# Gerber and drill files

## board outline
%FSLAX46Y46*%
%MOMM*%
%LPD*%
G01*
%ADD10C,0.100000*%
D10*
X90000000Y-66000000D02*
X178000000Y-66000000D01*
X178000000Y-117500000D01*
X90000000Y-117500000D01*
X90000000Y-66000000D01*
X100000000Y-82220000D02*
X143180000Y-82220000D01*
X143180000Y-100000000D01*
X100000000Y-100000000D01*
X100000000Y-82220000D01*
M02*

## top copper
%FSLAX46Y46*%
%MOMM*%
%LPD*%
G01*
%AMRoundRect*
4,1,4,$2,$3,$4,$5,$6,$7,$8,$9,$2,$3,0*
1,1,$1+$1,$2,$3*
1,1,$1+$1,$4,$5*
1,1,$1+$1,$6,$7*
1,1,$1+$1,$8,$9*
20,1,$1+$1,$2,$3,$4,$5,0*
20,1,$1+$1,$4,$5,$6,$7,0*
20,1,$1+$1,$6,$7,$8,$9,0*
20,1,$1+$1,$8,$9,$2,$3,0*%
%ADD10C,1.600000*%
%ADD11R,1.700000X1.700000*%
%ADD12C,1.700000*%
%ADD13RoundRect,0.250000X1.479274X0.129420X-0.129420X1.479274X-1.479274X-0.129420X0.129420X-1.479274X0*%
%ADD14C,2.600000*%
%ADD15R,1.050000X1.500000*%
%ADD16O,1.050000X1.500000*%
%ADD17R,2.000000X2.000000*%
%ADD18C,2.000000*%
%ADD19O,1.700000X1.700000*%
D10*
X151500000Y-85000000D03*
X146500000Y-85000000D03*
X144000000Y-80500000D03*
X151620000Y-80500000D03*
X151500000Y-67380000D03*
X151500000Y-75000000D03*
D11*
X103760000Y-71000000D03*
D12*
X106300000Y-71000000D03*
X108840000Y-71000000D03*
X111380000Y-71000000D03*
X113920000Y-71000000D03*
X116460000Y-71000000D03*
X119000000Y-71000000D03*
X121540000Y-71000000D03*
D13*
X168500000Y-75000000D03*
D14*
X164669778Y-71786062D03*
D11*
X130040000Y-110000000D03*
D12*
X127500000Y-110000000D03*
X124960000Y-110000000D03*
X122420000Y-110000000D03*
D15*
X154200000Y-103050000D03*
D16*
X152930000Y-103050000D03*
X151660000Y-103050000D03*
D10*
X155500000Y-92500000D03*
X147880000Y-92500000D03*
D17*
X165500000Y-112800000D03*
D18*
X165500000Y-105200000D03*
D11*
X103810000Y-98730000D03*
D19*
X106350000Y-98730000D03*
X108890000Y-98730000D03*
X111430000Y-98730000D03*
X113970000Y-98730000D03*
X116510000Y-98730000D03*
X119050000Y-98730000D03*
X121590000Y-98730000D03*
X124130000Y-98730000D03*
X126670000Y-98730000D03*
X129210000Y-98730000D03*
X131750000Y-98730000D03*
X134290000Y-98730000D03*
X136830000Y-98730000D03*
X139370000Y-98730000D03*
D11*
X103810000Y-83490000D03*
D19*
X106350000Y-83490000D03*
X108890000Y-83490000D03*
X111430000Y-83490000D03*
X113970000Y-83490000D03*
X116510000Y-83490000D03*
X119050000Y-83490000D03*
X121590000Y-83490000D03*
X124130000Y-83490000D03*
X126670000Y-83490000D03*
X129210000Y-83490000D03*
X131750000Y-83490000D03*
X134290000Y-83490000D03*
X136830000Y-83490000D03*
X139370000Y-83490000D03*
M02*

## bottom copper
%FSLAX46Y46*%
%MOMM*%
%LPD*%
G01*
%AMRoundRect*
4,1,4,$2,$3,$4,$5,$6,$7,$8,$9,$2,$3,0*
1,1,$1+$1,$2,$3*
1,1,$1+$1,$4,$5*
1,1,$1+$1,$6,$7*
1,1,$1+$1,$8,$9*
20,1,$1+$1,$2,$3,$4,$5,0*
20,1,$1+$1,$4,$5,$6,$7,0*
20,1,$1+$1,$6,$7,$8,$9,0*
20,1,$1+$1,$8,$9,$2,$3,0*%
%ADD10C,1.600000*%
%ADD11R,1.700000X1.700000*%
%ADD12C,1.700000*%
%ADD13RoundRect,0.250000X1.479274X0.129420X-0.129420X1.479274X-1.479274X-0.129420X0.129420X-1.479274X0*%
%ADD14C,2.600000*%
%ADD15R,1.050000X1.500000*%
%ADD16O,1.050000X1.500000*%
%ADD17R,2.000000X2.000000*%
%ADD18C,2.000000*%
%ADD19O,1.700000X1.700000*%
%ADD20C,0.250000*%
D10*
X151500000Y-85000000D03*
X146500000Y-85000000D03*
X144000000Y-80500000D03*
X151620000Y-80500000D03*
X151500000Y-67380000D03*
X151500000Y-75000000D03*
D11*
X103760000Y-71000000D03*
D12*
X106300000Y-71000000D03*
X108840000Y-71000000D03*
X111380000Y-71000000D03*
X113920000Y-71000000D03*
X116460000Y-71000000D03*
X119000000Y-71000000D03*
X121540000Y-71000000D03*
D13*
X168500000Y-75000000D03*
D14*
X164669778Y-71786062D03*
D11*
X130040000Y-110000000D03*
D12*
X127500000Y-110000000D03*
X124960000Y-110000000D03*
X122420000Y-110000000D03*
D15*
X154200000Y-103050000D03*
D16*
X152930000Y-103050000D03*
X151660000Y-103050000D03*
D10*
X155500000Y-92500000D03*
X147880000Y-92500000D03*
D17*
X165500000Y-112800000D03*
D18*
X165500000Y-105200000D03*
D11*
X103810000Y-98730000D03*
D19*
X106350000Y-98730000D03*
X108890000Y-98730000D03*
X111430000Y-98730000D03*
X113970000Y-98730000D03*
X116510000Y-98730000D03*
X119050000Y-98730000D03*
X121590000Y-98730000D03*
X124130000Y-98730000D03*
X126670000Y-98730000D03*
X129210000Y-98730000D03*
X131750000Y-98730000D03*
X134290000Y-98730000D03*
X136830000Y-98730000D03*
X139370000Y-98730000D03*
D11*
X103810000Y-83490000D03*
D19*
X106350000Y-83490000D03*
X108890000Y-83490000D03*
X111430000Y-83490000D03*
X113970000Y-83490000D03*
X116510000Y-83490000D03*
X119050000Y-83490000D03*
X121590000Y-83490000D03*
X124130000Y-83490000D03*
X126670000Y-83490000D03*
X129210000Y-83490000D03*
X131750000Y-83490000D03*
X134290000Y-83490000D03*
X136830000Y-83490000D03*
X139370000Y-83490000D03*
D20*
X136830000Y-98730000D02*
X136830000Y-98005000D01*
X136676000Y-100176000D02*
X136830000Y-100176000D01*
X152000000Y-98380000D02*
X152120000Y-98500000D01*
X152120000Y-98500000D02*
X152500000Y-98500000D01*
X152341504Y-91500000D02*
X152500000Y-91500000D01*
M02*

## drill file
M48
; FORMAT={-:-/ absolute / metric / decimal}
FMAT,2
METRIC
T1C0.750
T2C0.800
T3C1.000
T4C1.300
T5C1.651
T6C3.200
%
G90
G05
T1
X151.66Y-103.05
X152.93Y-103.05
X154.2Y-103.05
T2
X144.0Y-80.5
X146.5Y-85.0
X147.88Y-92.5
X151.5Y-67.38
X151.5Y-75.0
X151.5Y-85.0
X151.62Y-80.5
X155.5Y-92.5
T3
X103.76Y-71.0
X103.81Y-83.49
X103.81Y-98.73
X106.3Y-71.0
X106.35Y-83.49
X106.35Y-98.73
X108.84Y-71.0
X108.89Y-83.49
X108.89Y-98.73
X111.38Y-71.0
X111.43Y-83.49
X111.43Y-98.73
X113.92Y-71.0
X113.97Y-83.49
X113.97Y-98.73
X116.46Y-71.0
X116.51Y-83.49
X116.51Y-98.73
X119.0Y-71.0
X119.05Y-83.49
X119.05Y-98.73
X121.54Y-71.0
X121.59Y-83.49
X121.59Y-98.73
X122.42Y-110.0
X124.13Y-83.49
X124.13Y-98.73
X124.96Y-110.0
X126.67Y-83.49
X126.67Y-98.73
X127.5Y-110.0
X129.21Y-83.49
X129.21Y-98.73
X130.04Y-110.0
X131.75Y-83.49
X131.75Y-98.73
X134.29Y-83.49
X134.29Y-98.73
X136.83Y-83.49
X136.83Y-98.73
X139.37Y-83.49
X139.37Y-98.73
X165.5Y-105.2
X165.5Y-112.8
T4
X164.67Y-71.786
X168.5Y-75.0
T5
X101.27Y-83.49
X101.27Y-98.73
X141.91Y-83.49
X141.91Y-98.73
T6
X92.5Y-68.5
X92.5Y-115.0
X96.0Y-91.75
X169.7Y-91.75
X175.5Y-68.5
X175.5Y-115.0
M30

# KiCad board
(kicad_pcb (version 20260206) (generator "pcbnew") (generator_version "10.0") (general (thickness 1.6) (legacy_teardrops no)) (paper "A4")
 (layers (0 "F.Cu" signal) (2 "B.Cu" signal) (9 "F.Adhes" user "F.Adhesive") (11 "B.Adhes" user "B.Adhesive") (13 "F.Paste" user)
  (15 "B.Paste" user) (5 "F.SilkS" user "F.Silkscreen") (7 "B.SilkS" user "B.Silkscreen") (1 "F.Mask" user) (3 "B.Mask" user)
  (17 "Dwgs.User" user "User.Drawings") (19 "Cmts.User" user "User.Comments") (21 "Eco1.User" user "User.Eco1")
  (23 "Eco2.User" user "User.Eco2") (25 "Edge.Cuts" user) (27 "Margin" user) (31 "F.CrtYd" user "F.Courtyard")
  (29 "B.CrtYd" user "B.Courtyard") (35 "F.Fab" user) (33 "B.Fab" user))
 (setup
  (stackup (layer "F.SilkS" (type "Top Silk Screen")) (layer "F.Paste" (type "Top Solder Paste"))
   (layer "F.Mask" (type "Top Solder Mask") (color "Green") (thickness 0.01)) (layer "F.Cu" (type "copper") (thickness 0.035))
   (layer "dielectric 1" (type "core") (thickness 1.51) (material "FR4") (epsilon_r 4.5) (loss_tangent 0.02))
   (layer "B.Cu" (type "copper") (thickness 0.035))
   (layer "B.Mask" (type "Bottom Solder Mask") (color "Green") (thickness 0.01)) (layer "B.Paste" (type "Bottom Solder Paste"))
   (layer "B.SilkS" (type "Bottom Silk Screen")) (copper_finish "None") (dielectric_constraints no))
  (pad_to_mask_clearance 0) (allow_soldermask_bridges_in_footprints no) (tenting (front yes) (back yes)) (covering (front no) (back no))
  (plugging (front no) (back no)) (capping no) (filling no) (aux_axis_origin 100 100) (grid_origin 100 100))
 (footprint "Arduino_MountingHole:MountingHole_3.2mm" (layer "F.Cu") (at 96 91.75)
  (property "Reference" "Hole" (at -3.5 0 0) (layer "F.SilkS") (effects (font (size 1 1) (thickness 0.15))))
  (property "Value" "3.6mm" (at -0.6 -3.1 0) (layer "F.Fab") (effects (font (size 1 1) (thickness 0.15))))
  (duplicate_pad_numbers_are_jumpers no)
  (pad "" np_thru_hole circle (at 0 0) (size 3.2 3.2) (drill 3.2) (layers "*.Cu" "*.Mask")))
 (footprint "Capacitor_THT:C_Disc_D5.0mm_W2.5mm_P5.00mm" (layer "F.Cu") (at 151.5 85 180)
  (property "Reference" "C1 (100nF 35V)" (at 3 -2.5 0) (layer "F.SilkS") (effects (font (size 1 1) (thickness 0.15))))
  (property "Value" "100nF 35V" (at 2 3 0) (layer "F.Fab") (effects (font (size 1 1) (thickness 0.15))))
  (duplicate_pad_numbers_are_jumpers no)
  (pad "1" thru_hole circle (at 0 0 180) (size 1.6 1.6) (drill 0.8) (layers "*.Cu" "*.Mask") (remove_unused_layers no) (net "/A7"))
  (pad "2" thru_hole circle (at 5 0 180) (size 1.6 1.6) (drill 0.8) (layers "*.Cu" "*.Mask") (remove_unused_layers no) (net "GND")))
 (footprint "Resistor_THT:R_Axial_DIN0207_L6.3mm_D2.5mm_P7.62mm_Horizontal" (layer "F.Cu") (at 144 80.5)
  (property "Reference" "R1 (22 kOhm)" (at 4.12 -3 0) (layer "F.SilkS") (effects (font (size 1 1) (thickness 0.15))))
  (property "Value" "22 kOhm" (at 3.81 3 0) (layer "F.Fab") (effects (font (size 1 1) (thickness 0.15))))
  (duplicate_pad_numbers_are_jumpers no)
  (pad "1" thru_hole circle (at 0 0) (size 1.6 1.6) (drill 0.8) (layers "*.Cu" "*.Mask") (remove_unused_layers no) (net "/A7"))
  (pad "2" thru_hole circle (at 7.62 0) (size 1.6 1.6) (drill 0.8) (layers "*.Cu" "*.Mask") (remove_unused_layers no) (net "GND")))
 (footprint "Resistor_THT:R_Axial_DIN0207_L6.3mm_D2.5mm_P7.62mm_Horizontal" (layer "F.Cu") (at 151.5 67.38 -90)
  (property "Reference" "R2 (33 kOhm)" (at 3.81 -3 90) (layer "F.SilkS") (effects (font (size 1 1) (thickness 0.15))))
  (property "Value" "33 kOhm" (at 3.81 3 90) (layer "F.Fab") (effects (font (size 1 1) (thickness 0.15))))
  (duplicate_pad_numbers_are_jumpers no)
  (pad "1" thru_hole circle (at 0 0 270) (size 1.6 1.6) (drill 0.8) (layers "*.Cu" "*.Mask") (remove_unused_layers no) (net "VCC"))
  (pad "2" thru_hole circle (at 7.62 0 270) (size 1.6 1.6) (drill 0.8) (layers "*.Cu" "*.Mask") (remove_unused_layers no) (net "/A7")))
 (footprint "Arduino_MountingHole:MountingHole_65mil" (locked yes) (layer "F.Cu") (at 101.27 83.49)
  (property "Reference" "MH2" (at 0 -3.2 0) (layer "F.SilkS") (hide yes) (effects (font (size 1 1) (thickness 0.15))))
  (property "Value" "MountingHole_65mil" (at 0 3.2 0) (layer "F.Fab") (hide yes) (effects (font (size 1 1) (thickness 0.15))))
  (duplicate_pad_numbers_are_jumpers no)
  (pad "" np_thru_hole circle (at 0 0) (size 1.651 1.651) (drill 1.651) (layers "*.Cu" "*.Mask")))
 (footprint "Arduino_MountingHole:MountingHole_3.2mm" (layer "F.Cu") (at 92.5 115)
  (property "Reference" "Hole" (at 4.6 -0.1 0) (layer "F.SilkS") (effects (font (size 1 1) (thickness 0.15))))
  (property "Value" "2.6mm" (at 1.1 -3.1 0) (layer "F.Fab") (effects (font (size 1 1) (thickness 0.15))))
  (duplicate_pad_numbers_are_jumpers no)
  (pad "" np_thru_hole circle (at 0 0) (size 3.2 3.2) (drill 3.2) (layers "*.Cu" "*.Mask")))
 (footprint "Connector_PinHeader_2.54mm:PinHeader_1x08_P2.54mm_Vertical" (layer "F.Cu") (at 103.76 71 90)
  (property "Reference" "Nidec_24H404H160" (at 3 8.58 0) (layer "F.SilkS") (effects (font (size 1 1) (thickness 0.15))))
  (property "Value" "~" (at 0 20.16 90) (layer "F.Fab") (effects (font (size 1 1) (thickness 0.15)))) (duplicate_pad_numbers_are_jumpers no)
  (pad "1" thru_hole rect (at 0 0 90) (size 1.7 1.7) (drill 1) (layers "*.Cu" "*.Mask") (remove_unused_layers no) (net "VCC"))
  (pad "2" thru_hole circle (at 0 2.54 90) (size 1.7 1.7) (drill 1) (layers "*.Cu" "*.Mask") (remove_unused_layers no) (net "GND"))
  (pad "3" thru_hole circle (at 0 5.08 90) (size 1.7 1.7) (drill 1) (layers "*.Cu" "*.Mask") (remove_unused_layers no) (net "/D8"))
  (pad "4" thru_hole circle (at 0 7.62 90) (size 1.7 1.7) (drill 1) (layers "*.Cu" "*.Mask") (remove_unused_layers no) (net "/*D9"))
  (pad "5" thru_hole circle (at 0 10.16 90) (size 1.7 1.7) (drill 1) (layers "*.Cu" "*.Mask") (remove_unused_layers no) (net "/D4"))
  (pad "6" thru_hole circle (at 0 12.7 90) (size 1.7 1.7) (drill 1) (layers "*.Cu" "*.Mask") (remove_unused_layers no)
   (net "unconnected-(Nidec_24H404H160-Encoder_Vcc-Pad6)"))
  (pad "7" thru_hole circle (at 0 15.24 90) (size 1.7 1.7) (drill 1) (layers "*.Cu" "*.Mask") (remove_unused_layers no)
   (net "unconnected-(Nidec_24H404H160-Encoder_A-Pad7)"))
  (pad "8" thru_hole circle (at 0 17.78 90) (size 1.7 1.7) (drill 1) (layers "*.Cu" "*.Mask") (remove_unused_layers no)
   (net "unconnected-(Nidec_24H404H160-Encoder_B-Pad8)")))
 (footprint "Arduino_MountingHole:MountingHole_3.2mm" (layer "F.Cu") (at 175.5 68.5)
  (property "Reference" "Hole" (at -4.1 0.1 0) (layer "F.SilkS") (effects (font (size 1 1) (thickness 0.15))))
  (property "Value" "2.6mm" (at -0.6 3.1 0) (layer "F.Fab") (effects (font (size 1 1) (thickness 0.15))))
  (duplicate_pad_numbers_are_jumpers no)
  (pad "" np_thru_hole circle (at 0 0) (size 3.2 3.2) (drill 3.2) (layers "*.Cu" "*.Mask")))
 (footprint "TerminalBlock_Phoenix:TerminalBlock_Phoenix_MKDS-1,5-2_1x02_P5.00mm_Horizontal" (layer "F.Cu") (at 168.5 75 140)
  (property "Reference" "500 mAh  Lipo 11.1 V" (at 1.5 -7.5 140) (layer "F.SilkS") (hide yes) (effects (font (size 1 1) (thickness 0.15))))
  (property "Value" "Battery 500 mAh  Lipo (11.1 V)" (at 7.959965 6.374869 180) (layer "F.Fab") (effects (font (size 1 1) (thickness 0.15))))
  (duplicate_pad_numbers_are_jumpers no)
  (pad "1" thru_hole roundrect (at 0 0 140) (size 2.6 2.6) (drill 1.3) (layers "*.Cu" "*.Mask") (remove_unused_layers no)
   (roundrect_rratio 0.096154) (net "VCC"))
  (pad "2" thru_hole circle (at 5 0 140) (size 2.6 2.6) (drill 1.3) (layers "*.Cu" "*.Mask") (remove_unused_layers no) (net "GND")))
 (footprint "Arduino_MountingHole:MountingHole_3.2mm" (layer "F.Cu") (at 175.5 115)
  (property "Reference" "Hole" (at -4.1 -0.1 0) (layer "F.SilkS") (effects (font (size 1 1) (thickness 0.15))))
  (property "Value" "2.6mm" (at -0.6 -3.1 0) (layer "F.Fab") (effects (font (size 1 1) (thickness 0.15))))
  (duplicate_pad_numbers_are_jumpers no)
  (pad "" np_thru_hole circle (at 0 0) (size 3.2 3.2) (drill 3.2) (layers "*.Cu" "*.Mask")))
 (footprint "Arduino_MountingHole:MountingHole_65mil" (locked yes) (layer "F.Cu") (at 141.91 98.73)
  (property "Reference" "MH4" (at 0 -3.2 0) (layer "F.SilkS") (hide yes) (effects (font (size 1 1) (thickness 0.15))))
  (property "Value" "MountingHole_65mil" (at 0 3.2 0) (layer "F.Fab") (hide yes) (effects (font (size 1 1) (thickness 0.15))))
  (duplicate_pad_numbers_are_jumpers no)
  (pad "" np_thru_hole circle (at 0 0) (size 1.651 1.651) (drill 1.651) (layers "*.Cu" "*.Mask")))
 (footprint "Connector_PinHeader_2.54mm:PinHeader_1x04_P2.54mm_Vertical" (layer "F.Cu") (at 130.04 110 -90)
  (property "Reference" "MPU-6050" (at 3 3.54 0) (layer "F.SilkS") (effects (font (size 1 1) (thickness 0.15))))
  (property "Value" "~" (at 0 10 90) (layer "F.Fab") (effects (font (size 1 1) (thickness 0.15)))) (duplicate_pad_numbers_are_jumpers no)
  (pad "1" thru_hole rect (at 0 0 270) (size 1.7 1.7) (drill 1) (layers "*.Cu" "*.Mask") (remove_unused_layers no) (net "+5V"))
  (pad "2" thru_hole circle (at 0 2.54 270) (size 1.7 1.7) (drill 1) (layers "*.Cu" "*.Mask") (remove_unused_layers no) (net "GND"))
  (pad "3" thru_hole circle (at 0 5.08 270) (size 1.7 1.7) (drill 1) (layers "*.Cu" "*.Mask") (remove_unused_layers no)
   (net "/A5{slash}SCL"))
  (pad "4" thru_hole circle (at 0 7.62 270) (size 1.7 1.7) (drill 1) (layers "*.Cu" "*.Mask") (remove_unused_layers no)
   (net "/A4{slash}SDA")))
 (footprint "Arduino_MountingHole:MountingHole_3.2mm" (layer "F.Cu") (at 169.7 91.75)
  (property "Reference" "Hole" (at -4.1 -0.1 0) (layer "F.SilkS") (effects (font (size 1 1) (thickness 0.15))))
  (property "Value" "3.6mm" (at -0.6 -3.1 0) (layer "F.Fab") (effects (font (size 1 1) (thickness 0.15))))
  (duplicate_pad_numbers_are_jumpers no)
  (pad "" np_thru_hole circle (at 0 0) (size 3.2 3.2) (drill 3.2) (layers "*.Cu" "*.Mask")))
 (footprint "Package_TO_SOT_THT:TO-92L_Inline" (layer "F.Cu") (at 154.2 103.05 180)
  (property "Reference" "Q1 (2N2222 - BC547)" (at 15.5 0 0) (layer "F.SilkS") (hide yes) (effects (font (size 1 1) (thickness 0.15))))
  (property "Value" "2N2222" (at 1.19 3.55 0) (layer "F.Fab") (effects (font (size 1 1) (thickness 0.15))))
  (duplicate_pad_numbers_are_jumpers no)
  (pad "1" thru_hole rect (at 0 0 180) (size 1.05 1.5) (drill 0.75) (layers "*.Cu" "*.Mask") (remove_unused_layers no) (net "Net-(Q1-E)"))
  (pad "2" thru_hole oval (at 1.27 0 180) (size 1.05 1.5) (drill 0.75) (layers "*.Cu" "*.Mask") (remove_unused_layers no) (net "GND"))
  (pad "3" thru_hole oval (at 2.54 0 180) (size 1.05 1.5) (drill 0.75) (layers "*.Cu" "*.Mask") (remove_unused_layers no)
   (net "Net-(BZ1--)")))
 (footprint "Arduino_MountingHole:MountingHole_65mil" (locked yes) (layer "F.Cu") (at 101.27 98.73)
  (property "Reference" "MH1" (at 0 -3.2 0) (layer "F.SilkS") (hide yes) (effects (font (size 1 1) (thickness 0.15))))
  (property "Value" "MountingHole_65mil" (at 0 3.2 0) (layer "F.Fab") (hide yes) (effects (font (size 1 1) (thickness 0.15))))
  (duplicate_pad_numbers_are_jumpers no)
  (pad "" np_thru_hole circle (at 0 0) (size 1.651 1.651) (drill 1.651) (layers "*.Cu" "*.Mask")))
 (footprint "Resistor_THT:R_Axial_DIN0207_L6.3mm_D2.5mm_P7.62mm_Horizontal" (layer "F.Cu") (at 155.5 92.5 180)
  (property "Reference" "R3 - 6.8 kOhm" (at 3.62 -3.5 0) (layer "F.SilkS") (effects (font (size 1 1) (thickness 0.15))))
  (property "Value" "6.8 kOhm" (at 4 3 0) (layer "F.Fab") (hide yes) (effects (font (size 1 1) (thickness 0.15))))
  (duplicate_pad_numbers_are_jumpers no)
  (pad "1" thru_hole circle (at 0 0 180) (size 1.6 1.6) (drill 0.8) (layers "*.Cu" "*.Mask") (remove_unused_layers no) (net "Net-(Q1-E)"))
  (pad "2" thru_hole circle (at 7.62 0 180) (size 1.6 1.6) (drill 0.8) (layers "*.Cu" "*.Mask") (remove_unused_layers no)
   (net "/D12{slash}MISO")))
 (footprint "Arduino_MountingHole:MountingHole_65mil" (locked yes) (layer "F.Cu") (at 141.91 83.49)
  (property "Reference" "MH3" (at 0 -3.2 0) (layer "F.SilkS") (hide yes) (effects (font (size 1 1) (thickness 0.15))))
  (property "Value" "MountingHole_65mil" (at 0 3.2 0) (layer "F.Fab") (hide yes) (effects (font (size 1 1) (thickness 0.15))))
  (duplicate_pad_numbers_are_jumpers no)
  (pad "" np_thru_hole circle (at 0 0) (size 1.651 1.651) (drill 1.651) (layers "*.Cu" "*.Mask")))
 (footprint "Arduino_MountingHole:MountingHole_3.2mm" (layer "F.Cu") (at 92.5 68.5)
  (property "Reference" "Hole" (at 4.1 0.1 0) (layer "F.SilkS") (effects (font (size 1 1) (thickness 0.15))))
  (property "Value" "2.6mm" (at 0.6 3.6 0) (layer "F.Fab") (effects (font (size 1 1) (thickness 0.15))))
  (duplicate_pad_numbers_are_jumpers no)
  (pad "" np_thru_hole circle (at 0 0) (size 3.2 3.2) (drill 3.2) (layers "*.Cu" "*.Mask")))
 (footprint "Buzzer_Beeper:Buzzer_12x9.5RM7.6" (layer "F.Cu") (at 165.5 112.8 90)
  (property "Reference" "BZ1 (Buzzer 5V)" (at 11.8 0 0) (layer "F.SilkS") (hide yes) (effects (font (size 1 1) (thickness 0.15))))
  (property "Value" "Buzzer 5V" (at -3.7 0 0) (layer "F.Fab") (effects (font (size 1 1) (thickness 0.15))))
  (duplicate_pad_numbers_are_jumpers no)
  (pad "1" thru_hole rect (at 0 0 90) (size 2 2) (drill 1) (layers "*.Cu" "*.Mask") (remove_unused_layers no) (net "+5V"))
  (pad "2" thru_hole circle (at 7.6 0 90) (size 2 2) (drill 1) (layers "*.Cu" "*.Mask") (remove_unused_layers no) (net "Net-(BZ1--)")))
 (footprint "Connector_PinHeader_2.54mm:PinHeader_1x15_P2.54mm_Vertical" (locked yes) (layer "B.Cu") (at 103.81 98.73 -90)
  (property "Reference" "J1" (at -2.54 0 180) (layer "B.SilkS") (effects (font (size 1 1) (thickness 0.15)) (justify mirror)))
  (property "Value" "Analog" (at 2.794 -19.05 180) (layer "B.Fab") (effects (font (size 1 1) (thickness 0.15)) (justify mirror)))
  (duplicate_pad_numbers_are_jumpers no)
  (pad "1" thru_hole rect (at 0 0 270) (size 1.7 1.7) (drill 1) (layers "*.Cu" "*.Mask") (remove_unused_layers no) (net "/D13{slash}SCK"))
  (pad "2" thru_hole oval (at 0 -2.54 270) (size 1.7 1.7) (drill 1) (layers "*.Cu" "*.Mask") (remove_unused_layers no) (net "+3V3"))
  (pad "3" thru_hole oval (at 0 -5.08 270) (size 1.7 1.7) (drill 1) (layers "*.Cu" "*.Mask") (remove_unused_layers no) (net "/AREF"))
  (pad "4" thru_hole oval (at 0 -7.62 270) (size 1.7 1.7) (drill 1) (layers "*.Cu" "*.Mask") (remove_unused_layers no) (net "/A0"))
  (pad "5" thru_hole oval (at 0 -10.16 270) (size 1.7 1.7) (drill 1) (layers "*.Cu" "*.Mask") (remove_unused_layers no) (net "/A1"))
  (pad "6" thru_hole oval (at 0 -12.7 270) (size 1.7 1.7) (drill 1) (layers "*.Cu" "*.Mask") (remove_unused_layers no) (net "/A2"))
  (pad "7" thru_hole oval (at 0 -15.24 270) (size 1.7 1.7) (drill 1) (layers "*.Cu" "*.Mask") (remove_unused_layers no) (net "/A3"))
  (pad "8" thru_hole oval (at 0 -17.78 270) (size 1.7 1.7) (drill 1) (layers "*.Cu" "*.Mask") (remove_unused_layers no)
   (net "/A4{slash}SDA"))
  (pad "9" thru_hole oval (at 0 -20.32 270) (size 1.7 1.7) (drill 1) (layers "*.Cu" "*.Mask") (remove_unused_layers no)
   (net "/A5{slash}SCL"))
  (pad "10" thru_hole oval (at 0 -22.86 270) (size 1.7 1.7) (drill 1) (layers "*.Cu" "*.Mask") (remove_unused_layers no) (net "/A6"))
  (pad "11" thru_hole oval (at 0 -25.4 270) (size 1.7 1.7) (drill 1) (layers "*.Cu" "*.Mask") (remove_unused_layers no) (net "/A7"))
  (pad "12" thru_hole oval (at 0 -27.94 270) (size 1.7 1.7) (drill 1) (layers "*.Cu" "*.Mask") (remove_unused_layers no) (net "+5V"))
  (pad "13" thru_hole oval (at 0 -30.48 270) (size 1.7 1.7) (drill 1) (layers "*.Cu" "*.Mask") (remove_unused_layers no) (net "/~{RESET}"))
  (pad "14" thru_hole oval (at 0 -33.02 270) (size 1.7 1.7) (drill 1) (layers "*.Cu" "*.Mask") (remove_unused_layers no) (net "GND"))
  (pad "15" thru_hole oval (at 0 -35.56 270) (size 1.7 1.7) (drill 1) (layers "*.Cu" "*.Mask") (remove_unused_layers no) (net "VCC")))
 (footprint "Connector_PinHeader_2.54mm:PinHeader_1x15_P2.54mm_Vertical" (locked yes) (layer "B.Cu") (at 103.81 83.49 -90)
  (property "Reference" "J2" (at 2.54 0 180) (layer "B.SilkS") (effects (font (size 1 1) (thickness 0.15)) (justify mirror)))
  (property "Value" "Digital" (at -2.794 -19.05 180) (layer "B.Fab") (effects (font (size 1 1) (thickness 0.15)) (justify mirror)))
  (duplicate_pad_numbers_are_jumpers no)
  (pad "1" thru_hole rect (at 0 0 270) (size 1.7 1.7) (drill 1) (layers "*.Cu" "*.Mask") (remove_unused_layers no) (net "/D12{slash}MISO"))
  (pad "2" thru_hole oval (at 0 -2.54 270) (size 1.7 1.7) (drill 1) (layers "*.Cu" "*.Mask") (remove_unused_layers no)
   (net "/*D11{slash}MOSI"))
  (pad "3" thru_hole oval (at 0 -5.08 270) (size 1.7 1.7) (drill 1) (layers "*.Cu" "*.Mask") (remove_unused_layers no)
   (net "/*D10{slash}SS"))
  (pad "4" thru_hole oval (at 0 -7.62 270) (size 1.7 1.7) (drill 1) (layers "*.Cu" "*.Mask") (remove_unused_layers no) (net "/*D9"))
  (pad "5" thru_hole oval (at 0 -10.16 270) (size 1.7 1.7) (drill 1) (layers "*.Cu" "*.Mask") (remove_unused_layers no) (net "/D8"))
  (pad "6" thru_hole oval (at 0 -12.7 270) (size 1.7 1.7) (drill 1) (layers "*.Cu" "*.Mask") (remove_unused_layers no) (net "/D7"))
  (pad "7" thru_hole oval (at 0 -15.24 270) (size 1.7 1.7) (drill 1) (layers "*.Cu" "*.Mask") (remove_unused_layers no) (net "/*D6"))
  (pad "8" thru_hole oval (at 0 -17.78 270) (size 1.7 1.7) (drill 1) (layers "*.Cu" "*.Mask") (remove_unused_layers no) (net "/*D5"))
  (pad "9" thru_hole oval (at 0 -20.32 270) (size 1.7 1.7) (drill 1) (layers "*.Cu" "*.Mask") (remove_unused_layers no) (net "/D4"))
  (pad "10" thru_hole oval (at 0 -22.86 270) (size 1.7 1.7) (drill 1) (layers "*.Cu" "*.Mask") (remove_unused_layers no) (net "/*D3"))
  (pad "11" thru_hole oval (at 0 -25.4 270) (size 1.7 1.7) (drill 1) (layers "*.Cu" "*.Mask") (remove_unused_layers no) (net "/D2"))
  (pad "12" thru_hole oval (at 0 -27.94 270) (size 1.7 1.7) (drill 1) (layers "*.Cu" "*.Mask") (remove_unused_layers no) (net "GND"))
  (pad "13" thru_hole oval (at 0 -30.48 270) (size 1.7 1.7) (drill 1) (layers "*.Cu" "*.Mask") (remove_unused_layers no) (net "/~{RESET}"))
  (pad "14" thru_hole oval (at 0 -33.02 270) (size 1.7 1.7) (drill 1) (layers "*.Cu" "*.Mask") (remove_unused_layers no)
   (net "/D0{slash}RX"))
  (pad "15" thru_hole oval (at 0 -35.56 270) (size 1.7 1.7) (drill 1) (layers "*.Cu" "*.Mask") (remove_unused_layers no)
   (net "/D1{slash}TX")))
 (gr_rect (start 90 66) (end 178 117.5) (stroke (width 0.1) (type solid)) (fill no) (layer "Edge.Cuts"))
 (gr_rect (start 100 82.22) (end 143.18 100) (stroke (width 0.1) (type solid)) (fill no) (layer "Edge.Cuts"))
 (segment (start 136.83 98.73) (end 136.83 98.005) (width 0.25) (layer "B.Cu") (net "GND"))
 (segment (start 136.676 100.176) (end 136.83 100.176) (width 0.25) (layer "B.Cu") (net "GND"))
 (segment (start 152 98.38) (end 152.12 98.5) (width 0.25) (layer "B.Cu") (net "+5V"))
 (segment (start 152.12 98.5) (end 152.5 98.5) (width 0.25) (layer "B.Cu") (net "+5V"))
 (segment (start 152.341504 91.5) (end 152.5 91.5) (width 0.25) (layer "B.Cu") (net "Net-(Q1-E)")))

